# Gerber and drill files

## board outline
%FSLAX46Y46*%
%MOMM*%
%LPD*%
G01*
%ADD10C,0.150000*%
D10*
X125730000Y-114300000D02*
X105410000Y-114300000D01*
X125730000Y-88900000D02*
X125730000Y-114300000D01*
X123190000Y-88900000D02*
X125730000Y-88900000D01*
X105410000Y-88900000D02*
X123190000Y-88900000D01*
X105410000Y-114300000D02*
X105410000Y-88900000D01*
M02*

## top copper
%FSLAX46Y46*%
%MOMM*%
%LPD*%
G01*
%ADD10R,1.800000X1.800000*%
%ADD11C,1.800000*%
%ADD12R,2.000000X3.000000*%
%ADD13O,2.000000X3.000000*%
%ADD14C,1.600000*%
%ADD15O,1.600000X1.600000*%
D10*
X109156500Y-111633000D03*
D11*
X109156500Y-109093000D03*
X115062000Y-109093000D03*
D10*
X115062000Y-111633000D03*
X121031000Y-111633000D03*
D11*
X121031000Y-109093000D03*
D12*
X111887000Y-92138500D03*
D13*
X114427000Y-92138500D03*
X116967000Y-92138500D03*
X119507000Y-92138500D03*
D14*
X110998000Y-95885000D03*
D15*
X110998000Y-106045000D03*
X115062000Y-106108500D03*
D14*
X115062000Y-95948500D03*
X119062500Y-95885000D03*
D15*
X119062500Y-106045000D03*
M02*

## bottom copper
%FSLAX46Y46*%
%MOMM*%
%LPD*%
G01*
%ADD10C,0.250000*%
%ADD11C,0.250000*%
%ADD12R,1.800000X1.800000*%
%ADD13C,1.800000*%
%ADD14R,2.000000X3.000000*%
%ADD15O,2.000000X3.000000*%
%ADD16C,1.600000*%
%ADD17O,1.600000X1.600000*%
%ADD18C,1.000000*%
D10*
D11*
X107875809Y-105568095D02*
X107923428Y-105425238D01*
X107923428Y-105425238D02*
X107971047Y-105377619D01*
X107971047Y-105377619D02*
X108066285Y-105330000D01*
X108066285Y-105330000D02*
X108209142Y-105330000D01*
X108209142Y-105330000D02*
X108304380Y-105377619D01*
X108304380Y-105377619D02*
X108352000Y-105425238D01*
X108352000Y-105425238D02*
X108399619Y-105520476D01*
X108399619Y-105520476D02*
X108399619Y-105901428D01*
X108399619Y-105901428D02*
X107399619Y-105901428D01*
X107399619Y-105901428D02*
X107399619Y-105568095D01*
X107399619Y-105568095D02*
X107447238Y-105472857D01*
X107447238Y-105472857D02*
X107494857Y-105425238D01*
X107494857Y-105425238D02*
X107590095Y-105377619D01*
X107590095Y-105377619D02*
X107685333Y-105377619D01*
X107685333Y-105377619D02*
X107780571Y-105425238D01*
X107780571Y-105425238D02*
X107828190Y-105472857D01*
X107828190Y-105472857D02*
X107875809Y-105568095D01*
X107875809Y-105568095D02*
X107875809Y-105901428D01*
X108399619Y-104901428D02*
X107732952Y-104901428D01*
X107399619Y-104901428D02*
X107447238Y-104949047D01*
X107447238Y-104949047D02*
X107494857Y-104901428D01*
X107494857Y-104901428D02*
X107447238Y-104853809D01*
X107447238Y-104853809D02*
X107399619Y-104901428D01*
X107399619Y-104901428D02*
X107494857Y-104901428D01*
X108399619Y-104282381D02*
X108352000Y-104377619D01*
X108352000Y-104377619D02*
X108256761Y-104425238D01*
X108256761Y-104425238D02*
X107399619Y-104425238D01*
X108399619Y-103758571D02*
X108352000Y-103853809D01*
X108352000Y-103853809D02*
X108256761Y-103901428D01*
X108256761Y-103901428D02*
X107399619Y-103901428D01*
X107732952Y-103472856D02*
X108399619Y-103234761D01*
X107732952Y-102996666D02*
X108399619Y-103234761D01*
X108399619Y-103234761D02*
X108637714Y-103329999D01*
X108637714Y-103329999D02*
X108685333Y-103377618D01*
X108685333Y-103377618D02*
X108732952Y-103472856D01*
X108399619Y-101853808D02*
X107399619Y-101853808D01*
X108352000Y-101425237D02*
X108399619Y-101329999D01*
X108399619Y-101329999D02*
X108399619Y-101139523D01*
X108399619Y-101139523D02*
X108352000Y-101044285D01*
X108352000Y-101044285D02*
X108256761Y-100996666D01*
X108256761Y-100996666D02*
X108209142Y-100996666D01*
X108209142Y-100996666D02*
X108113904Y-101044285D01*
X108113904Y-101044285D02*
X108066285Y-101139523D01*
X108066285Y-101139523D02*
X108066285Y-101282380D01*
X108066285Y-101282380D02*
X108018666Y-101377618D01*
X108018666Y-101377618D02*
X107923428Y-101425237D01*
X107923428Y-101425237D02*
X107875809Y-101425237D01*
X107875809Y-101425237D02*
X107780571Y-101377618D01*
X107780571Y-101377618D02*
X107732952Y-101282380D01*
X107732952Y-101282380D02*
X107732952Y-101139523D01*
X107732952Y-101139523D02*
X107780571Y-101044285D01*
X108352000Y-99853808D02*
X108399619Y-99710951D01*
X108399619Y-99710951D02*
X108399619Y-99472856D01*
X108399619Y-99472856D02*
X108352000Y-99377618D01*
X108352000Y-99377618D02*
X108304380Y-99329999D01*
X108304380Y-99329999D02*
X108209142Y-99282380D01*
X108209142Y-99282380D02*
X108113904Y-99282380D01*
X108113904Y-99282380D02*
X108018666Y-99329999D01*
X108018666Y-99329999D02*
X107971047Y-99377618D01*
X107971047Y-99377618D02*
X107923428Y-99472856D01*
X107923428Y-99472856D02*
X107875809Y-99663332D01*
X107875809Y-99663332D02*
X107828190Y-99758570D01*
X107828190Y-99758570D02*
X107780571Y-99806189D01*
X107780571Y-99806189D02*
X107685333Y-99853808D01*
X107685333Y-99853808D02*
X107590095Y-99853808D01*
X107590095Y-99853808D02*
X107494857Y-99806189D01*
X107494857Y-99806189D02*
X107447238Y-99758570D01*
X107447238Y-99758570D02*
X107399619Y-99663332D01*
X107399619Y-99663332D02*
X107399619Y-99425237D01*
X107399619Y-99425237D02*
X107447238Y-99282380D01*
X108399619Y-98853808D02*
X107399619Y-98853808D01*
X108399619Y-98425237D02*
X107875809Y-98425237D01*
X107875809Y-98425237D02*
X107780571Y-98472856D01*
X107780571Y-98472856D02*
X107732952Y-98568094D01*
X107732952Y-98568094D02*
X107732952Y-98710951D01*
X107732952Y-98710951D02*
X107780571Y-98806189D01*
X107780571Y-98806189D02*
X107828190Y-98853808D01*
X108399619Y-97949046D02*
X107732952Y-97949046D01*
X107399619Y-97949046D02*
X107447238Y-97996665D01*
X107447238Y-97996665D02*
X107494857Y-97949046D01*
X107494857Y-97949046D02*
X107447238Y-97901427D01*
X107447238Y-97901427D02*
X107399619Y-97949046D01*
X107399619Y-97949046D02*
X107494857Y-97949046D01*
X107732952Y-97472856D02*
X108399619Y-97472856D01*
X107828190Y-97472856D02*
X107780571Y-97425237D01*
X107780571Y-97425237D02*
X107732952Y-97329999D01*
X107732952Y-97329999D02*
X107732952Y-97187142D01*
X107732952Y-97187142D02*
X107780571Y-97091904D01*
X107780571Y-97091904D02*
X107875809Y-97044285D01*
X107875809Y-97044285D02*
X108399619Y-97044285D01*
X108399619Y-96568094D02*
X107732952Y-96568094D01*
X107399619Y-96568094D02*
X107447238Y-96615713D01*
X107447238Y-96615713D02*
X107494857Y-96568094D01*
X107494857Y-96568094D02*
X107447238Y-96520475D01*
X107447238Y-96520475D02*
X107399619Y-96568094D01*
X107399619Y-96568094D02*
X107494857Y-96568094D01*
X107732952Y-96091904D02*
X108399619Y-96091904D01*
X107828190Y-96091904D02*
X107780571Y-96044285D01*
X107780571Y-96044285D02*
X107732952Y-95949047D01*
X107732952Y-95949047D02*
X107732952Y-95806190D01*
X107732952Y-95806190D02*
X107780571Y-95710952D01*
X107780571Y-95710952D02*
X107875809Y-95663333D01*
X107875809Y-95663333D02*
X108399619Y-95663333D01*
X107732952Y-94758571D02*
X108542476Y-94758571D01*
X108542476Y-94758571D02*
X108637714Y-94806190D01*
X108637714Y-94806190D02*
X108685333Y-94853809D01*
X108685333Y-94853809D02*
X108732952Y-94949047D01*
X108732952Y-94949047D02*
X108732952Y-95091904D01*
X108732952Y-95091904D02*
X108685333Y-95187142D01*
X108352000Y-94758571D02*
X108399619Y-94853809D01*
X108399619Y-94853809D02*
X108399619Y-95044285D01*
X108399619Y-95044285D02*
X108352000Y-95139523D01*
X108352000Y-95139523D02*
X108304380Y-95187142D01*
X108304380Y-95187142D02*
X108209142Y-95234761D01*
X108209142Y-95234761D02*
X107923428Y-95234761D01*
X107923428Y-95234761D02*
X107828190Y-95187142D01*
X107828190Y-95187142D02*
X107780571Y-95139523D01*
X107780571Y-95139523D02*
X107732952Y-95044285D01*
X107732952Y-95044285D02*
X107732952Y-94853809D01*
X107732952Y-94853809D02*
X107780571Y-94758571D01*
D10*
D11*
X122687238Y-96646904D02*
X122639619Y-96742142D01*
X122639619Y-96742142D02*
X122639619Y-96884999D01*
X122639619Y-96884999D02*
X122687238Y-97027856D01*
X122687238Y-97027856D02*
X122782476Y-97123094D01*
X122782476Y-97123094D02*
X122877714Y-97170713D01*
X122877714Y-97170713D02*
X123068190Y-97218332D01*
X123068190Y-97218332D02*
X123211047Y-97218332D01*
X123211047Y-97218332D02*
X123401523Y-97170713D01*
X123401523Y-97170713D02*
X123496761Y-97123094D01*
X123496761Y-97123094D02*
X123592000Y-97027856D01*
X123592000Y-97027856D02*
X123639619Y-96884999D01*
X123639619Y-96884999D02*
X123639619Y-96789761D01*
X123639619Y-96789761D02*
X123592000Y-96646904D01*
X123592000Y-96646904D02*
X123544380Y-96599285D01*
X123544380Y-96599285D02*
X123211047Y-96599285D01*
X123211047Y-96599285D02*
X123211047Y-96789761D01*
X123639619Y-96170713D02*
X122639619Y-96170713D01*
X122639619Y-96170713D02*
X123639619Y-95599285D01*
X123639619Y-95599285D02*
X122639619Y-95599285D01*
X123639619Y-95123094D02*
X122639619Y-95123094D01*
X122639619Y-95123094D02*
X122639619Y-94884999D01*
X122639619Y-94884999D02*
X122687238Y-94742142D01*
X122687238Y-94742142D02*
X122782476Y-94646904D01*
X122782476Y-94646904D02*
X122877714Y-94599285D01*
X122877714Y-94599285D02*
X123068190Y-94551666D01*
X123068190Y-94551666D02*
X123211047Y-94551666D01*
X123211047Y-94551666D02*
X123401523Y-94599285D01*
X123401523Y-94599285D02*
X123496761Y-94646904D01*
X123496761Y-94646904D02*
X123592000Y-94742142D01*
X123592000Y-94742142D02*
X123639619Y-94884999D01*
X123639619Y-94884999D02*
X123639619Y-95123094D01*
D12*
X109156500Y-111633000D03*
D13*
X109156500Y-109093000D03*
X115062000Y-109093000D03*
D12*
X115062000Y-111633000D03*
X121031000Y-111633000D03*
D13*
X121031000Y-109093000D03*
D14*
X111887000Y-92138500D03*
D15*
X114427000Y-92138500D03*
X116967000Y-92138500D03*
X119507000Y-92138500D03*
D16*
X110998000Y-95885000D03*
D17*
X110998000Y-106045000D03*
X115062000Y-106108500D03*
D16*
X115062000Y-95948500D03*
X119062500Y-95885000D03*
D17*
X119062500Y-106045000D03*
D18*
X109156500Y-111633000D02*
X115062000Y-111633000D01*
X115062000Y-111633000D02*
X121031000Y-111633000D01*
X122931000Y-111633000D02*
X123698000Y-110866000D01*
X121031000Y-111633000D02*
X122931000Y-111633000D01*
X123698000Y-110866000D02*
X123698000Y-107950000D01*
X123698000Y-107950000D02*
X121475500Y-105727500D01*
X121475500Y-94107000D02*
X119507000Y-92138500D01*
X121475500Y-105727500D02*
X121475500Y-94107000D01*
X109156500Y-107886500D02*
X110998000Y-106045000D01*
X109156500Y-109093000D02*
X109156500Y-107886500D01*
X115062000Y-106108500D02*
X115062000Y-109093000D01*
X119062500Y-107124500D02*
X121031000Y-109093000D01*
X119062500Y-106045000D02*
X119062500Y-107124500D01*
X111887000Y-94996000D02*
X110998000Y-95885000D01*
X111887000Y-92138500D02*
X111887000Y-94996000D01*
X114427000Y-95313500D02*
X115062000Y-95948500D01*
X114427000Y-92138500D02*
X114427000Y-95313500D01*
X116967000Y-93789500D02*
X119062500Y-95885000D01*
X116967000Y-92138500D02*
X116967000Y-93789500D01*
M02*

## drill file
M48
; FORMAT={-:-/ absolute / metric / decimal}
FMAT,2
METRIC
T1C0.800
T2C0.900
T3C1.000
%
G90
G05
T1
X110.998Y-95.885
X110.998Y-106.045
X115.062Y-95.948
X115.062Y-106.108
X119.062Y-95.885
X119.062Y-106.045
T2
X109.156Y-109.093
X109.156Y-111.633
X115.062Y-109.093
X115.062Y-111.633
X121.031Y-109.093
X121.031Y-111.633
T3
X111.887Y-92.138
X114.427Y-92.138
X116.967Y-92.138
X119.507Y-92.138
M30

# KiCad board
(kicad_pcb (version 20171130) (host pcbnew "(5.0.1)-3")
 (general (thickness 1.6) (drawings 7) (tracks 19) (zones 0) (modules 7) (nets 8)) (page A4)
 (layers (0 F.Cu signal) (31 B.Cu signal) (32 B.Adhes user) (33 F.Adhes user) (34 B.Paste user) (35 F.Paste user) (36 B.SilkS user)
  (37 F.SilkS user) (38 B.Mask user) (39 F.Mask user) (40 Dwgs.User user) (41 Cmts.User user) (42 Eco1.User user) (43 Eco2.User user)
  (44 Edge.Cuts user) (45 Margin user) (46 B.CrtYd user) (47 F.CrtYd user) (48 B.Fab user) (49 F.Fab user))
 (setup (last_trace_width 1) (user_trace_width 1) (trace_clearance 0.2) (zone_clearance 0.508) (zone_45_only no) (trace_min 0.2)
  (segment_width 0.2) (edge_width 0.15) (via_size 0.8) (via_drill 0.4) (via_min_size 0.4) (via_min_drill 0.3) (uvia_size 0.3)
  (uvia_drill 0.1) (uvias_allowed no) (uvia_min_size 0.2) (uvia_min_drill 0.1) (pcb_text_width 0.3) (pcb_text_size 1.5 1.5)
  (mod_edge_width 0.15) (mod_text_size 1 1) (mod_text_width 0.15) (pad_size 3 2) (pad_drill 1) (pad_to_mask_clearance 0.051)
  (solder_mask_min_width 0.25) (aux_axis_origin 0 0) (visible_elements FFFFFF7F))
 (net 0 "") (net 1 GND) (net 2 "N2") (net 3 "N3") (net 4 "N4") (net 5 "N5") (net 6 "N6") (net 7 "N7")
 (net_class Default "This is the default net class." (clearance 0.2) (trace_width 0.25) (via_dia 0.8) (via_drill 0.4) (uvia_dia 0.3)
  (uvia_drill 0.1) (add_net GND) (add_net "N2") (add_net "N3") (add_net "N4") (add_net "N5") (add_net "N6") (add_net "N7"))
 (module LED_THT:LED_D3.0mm (layer F.Cu) (at 109.1565 111.633 90)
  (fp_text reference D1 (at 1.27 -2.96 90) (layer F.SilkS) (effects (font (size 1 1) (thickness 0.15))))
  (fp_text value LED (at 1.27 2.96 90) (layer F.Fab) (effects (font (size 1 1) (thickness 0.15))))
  (pad 1 thru_hole rect (at 0 0 90) (size 1.8 1.8) (drill 0.9) (layers *.Cu *.Mask) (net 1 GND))
  (pad 2 thru_hole circle (at 2.54 0 90) (size 1.8 1.8) (drill 0.9) (layers *.Cu *.Mask) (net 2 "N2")))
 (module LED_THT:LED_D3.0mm (layer F.Cu) (at 115.062 111.633 90)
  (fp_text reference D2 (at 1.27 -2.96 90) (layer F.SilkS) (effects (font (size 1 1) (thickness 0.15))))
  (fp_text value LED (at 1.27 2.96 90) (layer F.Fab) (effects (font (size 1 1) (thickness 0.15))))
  (pad 2 thru_hole circle (at 2.54 0 90) (size 1.8 1.8) (drill 0.9) (layers *.Cu *.Mask) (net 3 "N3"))
  (pad 1 thru_hole rect (at 0 0 90) (size 1.8 1.8) (drill 0.9) (layers *.Cu *.Mask) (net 1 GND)))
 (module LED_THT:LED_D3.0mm (layer F.Cu) (at 121.031 111.633 90)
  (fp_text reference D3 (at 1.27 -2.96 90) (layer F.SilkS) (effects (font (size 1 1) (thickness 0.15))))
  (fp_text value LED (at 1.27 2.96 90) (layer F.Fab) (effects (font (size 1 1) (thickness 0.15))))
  (pad 1 thru_hole rect (at 0 0 90) (size 1.8 1.8) (drill 0.9) (layers *.Cu *.Mask) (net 1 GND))
  (pad 2 thru_hole circle (at 2.54 0 90) (size 1.8 1.8) (drill 0.9) (layers *.Cu *.Mask) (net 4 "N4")))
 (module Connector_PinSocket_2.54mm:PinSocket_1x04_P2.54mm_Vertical (layer F.Cu) (at 111.887 92.1385 90)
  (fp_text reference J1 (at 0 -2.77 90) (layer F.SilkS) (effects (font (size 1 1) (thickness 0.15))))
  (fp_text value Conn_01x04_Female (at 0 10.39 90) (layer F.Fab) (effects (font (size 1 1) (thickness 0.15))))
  (pad 1 thru_hole rect (at 0 0 90) (size 3 2) (drill 1) (layers *.Cu *.Mask) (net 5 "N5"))
  (pad 2 thru_hole oval (at 0 2.54 90) (size 3 2) (drill 1) (layers *.Cu *.Mask) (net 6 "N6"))
  (pad 3 thru_hole oval (at 0 5.08 90) (size 3 2) (drill 1) (layers *.Cu *.Mask) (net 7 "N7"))
  (pad 4 thru_hole oval (at 0 7.62 90) (size 3 2) (drill 1) (layers *.Cu *.Mask) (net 1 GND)))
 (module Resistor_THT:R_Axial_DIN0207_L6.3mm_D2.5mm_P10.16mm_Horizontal (layer F.Cu) (at 110.998 95.885 270)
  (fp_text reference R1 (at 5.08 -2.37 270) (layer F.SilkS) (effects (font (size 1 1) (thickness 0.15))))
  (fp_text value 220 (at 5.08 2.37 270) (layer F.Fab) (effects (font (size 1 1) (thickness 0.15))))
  (pad 1 thru_hole circle (at 0 0 270) (size 1.6 1.6) (drill 0.8) (layers *.Cu *.Mask) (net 5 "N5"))
  (pad 2 thru_hole oval (at 10.16 0 270) (size 1.6 1.6) (drill 0.8) (layers *.Cu *.Mask) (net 2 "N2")))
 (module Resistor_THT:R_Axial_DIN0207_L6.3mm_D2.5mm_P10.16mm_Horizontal (layer F.Cu) (at 115.062 95.9485 270)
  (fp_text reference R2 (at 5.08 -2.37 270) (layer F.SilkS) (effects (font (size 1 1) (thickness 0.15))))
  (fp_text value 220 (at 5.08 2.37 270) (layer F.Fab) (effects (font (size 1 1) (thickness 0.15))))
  (pad 2 thru_hole oval (at 10.16 0 270) (size 1.6 1.6) (drill 0.8) (layers *.Cu *.Mask) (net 3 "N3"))
  (pad 1 thru_hole circle (at 0 0 270) (size 1.6 1.6) (drill 0.8) (layers *.Cu *.Mask) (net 6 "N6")))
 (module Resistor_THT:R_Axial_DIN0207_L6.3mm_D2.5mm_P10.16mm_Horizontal (layer F.Cu) (at 119.0625 95.885 270)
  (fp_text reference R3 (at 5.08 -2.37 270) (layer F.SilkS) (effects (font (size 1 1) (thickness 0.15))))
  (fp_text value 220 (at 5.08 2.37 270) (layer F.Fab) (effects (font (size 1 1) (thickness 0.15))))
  (pad 1 thru_hole circle (at 0 0 270) (size 1.6 1.6) (drill 0.8) (layers *.Cu *.Mask) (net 7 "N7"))
  (pad 2 thru_hole oval (at 10.16 0 270) (size 1.6 1.6) (drill 0.8) (layers *.Cu *.Mask) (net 4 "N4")))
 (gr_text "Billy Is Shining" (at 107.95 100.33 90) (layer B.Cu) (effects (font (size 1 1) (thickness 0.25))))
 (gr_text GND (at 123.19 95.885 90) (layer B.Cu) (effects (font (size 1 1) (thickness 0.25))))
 (gr_line (start 125.73 114.3) (end 105.41 114.3) (layer Edge.Cuts) (width 0.15))
 (gr_line (start 125.73 88.9) (end 125.73 114.3) (layer Edge.Cuts) (width 0.15))
 (gr_line (start 123.19 88.9) (end 125.73 88.9) (layer Edge.Cuts) (width 0.15))
 (gr_line (start 105.41 88.9) (end 123.19 88.9) (layer Edge.Cuts) (width 0.15))
 (gr_line (start 105.41 114.3) (end 105.41 88.9) (layer Edge.Cuts) (width 0.15))
 (segment (start 109.1565 111.633) (end 115.062 111.633) (width 1) (layer B.Cu) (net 1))
 (segment (start 115.062 111.633) (end 121.031 111.633) (width 1) (layer B.Cu) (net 1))
 (segment (start 122.931 111.633) (end 123.698 110.866) (width 1) (layer B.Cu) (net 1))
 (segment (start 121.031 111.633) (end 122.931 111.633) (width 1) (layer B.Cu) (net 1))
 (segment (start 123.698 110.866) (end 123.698 107.95) (width 1) (layer B.Cu) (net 1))
 (segment (start 123.698 107.95) (end 121.4755 105.7275) (width 1) (layer B.Cu) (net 1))
 (segment (start 121.4755 94.107) (end 119.507 92.1385) (width 1) (layer B.Cu) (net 1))
 (segment (start 121.4755 105.7275) (end 121.4755 94.107) (width 1) (layer B.Cu) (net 1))
 (segment (start 109.1565 107.8865) (end 110.998 106.045) (width 1) (layer B.Cu) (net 2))
 (segment (start 109.1565 109.093) (end 109.1565 107.8865) (width 1) (layer B.Cu) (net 2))
 (segment (start 115.062 106.1085) (end 115.062 109.093) (width 1) (layer B.Cu) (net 3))
 (segment (start 119.0625 107.1245) (end 121.031 109.093) (width 1) (layer B.Cu) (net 4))
 (segment (start 119.0625 106.045) (end 119.0625 107.1245) (width 1) (layer B.Cu) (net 4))
 (segment (start 111.887 94.996) (end 110.998 95.885) (width 1) (layer B.Cu) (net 5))
 (segment (start 111.887 92.1385) (end 111.887 94.996) (width 1) (layer B.Cu) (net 5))
 (segment (start 114.427 95.3135) (end 115.062 95.9485) (width 1) (layer B.Cu) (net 6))
 (segment (start 114.427 92.1385) (end 114.427 95.3135) (width 1) (layer B.Cu) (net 6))
 (segment (start 116.967 93.7895) (end 119.0625 95.885) (width 1) (layer B.Cu) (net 7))
 (segment (start 116.967 92.1385) (end 116.967 93.7895) (width 1) (layer B.Cu) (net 7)))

